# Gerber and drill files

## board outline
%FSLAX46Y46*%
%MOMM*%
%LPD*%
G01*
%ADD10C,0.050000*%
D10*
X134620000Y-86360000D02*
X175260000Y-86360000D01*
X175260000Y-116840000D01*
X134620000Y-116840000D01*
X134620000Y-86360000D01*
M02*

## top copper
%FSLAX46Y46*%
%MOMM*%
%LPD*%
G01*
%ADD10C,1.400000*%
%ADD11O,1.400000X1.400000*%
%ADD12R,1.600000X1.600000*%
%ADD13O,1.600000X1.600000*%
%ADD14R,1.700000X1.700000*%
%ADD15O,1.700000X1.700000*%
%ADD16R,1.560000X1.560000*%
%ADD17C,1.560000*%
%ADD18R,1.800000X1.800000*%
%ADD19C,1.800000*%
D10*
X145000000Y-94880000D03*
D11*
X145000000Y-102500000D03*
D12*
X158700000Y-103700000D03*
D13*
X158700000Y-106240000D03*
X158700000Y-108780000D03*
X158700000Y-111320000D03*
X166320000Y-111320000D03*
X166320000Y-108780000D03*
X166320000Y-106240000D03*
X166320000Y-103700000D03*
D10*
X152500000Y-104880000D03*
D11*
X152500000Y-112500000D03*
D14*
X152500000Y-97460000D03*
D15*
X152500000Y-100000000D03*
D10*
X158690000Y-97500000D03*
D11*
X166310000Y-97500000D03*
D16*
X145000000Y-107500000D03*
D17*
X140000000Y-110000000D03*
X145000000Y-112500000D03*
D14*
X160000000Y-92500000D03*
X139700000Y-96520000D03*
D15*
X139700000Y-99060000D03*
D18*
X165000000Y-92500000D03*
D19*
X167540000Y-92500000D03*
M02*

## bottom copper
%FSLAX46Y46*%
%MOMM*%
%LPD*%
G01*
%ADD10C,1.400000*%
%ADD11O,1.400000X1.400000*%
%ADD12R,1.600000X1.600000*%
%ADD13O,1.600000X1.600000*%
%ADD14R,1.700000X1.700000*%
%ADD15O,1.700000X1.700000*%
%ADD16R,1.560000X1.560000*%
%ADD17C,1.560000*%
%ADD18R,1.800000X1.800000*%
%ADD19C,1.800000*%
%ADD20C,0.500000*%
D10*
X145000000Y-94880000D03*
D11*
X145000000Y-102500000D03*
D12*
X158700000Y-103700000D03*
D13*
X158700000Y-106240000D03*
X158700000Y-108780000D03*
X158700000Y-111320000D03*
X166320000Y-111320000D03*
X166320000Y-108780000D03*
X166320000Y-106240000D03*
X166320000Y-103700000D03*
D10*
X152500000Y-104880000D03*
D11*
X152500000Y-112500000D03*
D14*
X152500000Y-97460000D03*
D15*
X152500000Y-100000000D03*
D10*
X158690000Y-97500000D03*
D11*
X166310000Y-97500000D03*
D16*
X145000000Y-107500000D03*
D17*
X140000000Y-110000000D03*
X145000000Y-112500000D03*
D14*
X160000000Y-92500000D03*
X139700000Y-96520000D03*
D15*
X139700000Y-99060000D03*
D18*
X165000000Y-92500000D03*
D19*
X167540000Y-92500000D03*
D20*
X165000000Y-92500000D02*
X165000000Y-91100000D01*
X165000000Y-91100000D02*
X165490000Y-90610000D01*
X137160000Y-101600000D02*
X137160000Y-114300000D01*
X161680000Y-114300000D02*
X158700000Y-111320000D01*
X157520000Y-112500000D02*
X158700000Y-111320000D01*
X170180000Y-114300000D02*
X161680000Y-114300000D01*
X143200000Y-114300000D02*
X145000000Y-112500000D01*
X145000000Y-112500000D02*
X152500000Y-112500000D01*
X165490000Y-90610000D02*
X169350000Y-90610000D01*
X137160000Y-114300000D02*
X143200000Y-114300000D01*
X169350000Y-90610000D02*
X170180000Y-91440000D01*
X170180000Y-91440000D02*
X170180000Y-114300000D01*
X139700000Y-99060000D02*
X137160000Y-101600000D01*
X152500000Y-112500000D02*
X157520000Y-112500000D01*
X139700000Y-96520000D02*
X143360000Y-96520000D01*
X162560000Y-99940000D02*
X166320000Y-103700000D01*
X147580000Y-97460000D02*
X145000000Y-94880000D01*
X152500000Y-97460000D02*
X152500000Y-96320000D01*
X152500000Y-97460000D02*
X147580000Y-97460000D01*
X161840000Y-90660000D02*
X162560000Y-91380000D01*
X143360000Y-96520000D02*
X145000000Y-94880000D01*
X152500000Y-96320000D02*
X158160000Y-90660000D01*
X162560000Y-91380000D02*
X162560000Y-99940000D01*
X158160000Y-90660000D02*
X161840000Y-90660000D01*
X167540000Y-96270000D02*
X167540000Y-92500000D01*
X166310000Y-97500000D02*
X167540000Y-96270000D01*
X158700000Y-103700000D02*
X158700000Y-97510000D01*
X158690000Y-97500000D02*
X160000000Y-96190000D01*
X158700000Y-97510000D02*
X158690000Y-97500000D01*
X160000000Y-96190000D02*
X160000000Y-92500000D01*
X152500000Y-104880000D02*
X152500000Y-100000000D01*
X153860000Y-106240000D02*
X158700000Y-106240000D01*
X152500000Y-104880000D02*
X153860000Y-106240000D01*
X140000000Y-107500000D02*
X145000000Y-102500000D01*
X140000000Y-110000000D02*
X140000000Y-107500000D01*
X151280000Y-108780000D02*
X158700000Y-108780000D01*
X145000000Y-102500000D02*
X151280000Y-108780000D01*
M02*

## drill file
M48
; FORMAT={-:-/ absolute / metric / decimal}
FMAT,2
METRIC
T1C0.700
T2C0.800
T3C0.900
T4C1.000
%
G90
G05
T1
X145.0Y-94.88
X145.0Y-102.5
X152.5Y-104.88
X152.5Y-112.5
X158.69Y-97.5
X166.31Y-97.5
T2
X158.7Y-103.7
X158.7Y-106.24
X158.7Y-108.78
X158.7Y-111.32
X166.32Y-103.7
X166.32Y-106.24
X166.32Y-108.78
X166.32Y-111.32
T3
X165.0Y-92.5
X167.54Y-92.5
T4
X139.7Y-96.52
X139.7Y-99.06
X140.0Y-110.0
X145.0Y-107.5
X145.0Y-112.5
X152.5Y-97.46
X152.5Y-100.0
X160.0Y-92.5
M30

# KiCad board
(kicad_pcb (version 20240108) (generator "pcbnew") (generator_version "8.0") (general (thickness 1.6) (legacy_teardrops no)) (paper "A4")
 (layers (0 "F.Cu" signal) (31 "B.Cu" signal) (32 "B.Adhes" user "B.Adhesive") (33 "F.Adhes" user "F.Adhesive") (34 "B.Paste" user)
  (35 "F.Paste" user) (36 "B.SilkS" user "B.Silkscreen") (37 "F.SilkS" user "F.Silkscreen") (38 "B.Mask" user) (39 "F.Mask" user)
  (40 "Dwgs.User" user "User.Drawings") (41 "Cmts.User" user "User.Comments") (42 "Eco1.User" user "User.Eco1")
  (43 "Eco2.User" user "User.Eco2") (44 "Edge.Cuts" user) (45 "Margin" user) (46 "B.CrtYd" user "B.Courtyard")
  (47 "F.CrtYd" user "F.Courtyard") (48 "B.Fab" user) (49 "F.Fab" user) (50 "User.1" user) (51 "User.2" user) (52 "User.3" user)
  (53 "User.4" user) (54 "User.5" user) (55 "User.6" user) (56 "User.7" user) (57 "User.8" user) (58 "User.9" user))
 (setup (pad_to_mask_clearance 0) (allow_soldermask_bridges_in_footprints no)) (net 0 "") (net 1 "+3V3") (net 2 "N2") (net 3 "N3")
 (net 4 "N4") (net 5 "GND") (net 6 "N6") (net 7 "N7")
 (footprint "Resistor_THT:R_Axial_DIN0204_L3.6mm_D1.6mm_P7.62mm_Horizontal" (layer "F.Cu") (at 145 94.88 -90)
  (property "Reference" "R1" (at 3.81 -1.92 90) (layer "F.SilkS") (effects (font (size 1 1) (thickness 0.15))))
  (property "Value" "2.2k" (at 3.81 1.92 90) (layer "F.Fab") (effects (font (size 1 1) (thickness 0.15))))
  (pad "1" thru_hole circle (at 0 0 270) (size 1.4 1.4) (drill 0.7) (layers "*.Cu" "*.Mask") (remove_unused_layers no) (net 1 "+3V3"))
  (pad "2" thru_hole oval (at 7.62 0 270) (size 1.4 1.4) (drill 0.7) (layers "*.Cu" "*.Mask") (remove_unused_layers no) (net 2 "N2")))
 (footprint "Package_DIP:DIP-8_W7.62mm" (layer "F.Cu") (at 158.7 103.7)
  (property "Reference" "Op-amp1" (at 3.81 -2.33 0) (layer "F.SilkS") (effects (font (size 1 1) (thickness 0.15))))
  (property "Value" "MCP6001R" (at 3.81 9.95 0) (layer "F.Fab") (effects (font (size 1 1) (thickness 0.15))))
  (pad "1" thru_hole rect (at 0 0) (size 1.6 1.6) (drill 0.8) (layers "*.Cu" "*.Mask") (remove_unused_layers no) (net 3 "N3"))
  (pad "2" thru_hole oval (at 0 2.54) (size 1.6 1.6) (drill 0.8) (layers "*.Cu" "*.Mask") (remove_unused_layers no) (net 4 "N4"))
  (pad "3" thru_hole oval (at 0 5.08) (size 1.6 1.6) (drill 0.8) (layers "*.Cu" "*.Mask") (remove_unused_layers no) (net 2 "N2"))
  (pad "4" thru_hole oval (at 0 7.62) (size 1.6 1.6) (drill 0.8) (layers "*.Cu" "*.Mask") (remove_unused_layers no) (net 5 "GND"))
  (pad "5" thru_hole oval (at 7.62 7.62) (size 1.6 1.6) (drill 0.8) (layers "*.Cu" "*.Mask") (remove_unused_layers no))
  (pad "6" thru_hole oval (at 7.62 5.08) (size 1.6 1.6) (drill 0.8) (layers "*.Cu" "*.Mask") (remove_unused_layers no))
  (pad "7" thru_hole oval (at 7.62 2.54) (size 1.6 1.6) (drill 0.8) (layers "*.Cu" "*.Mask") (remove_unused_layers no))
  (pad "8" thru_hole oval (at 7.62 0) (size 1.6 1.6) (drill 0.8) (layers "*.Cu" "*.Mask") (remove_unused_layers no) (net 1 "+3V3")))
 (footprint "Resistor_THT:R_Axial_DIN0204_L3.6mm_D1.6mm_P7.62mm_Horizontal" (layer "F.Cu") (at 152.5 104.88 -90)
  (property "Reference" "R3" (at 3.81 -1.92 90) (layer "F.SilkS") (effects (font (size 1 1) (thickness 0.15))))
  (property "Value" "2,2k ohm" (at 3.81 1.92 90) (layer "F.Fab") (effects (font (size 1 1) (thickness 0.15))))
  (pad "1" thru_hole circle (at 0 0 270) (size 1.4 1.4) (drill 0.7) (layers "*.Cu" "*.Mask") (remove_unused_layers no) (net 4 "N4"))
  (pad "2" thru_hole oval (at 7.62 0 270) (size 1.4 1.4) (drill 0.7) (layers "*.Cu" "*.Mask") (remove_unused_layers no) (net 5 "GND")))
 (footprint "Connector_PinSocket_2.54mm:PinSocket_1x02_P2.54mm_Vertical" (layer "F.Cu") (at 152.5 97.46)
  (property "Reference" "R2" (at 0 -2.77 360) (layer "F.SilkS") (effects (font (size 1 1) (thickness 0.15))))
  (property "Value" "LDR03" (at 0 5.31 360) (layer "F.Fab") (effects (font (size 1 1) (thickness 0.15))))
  (pad "1" thru_hole rect (at 0 0) (size 1.7 1.7) (drill 1) (layers "*.Cu" "*.Mask") (remove_unused_layers no) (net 1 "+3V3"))
  (pad "2" thru_hole oval (at 0 2.54) (size 1.7 1.7) (drill 1) (layers "*.Cu" "*.Mask") (remove_unused_layers no) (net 4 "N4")))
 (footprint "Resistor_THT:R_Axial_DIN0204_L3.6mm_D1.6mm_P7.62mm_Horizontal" (layer "F.Cu") (at 158.69 97.5)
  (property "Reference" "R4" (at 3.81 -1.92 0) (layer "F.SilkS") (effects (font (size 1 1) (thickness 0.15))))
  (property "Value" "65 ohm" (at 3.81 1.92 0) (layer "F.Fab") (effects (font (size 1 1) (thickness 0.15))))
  (pad "1" thru_hole circle (at 0 0) (size 1.4 1.4) (drill 0.7) (layers "*.Cu" "*.Mask") (remove_unused_layers no) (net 3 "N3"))
  (pad "2" thru_hole oval (at 7.62 0) (size 1.4 1.4) (drill 0.7) (layers "*.Cu" "*.Mask") (remove_unused_layers no) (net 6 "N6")))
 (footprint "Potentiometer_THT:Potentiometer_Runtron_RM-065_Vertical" (layer "F.Cu") (at 145 107.5 -90)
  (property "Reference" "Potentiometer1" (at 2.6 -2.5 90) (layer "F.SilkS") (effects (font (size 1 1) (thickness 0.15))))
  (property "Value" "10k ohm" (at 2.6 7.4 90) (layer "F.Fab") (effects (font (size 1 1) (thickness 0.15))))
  (pad "1" thru_hole rect (at 0 0 270) (size 1.56 1.56) (drill 1) (layers "*.Cu" "*.Mask") (remove_unused_layers no) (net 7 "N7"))
  (pad "2" thru_hole circle (at 2.5 5 270) (size 1.56 1.56) (drill 1) (layers "*.Cu" "*.Mask") (remove_unused_layers no) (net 2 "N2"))
  (pad "3" thru_hole circle (at 5 0 270) (size 1.56 1.56) (drill 1) (layers "*.Cu" "*.Mask") (remove_unused_layers no) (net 5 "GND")))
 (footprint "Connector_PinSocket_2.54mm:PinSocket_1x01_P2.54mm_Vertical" (layer "F.Cu") (at 160 92.5)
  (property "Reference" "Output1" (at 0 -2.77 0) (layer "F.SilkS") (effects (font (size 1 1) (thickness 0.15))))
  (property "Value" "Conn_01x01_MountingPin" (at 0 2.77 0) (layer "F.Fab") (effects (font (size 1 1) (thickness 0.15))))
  (pad "1" thru_hole rect (at 0 0) (size 1.7 1.7) (drill 1) (layers "*.Cu" "*.Mask") (remove_unused_layers no) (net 3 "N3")))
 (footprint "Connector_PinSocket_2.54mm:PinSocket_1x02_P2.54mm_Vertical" (layer "F.Cu") (at 139.7 96.52)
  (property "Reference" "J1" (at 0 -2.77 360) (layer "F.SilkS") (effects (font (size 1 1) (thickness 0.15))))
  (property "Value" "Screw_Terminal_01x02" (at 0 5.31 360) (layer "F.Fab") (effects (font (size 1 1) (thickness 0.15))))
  (pad "1" thru_hole rect (at 0 0) (size 1.7 1.7) (drill 1) (layers "*.Cu" "*.Mask") (remove_unused_layers no) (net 1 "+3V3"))
  (pad "2" thru_hole oval (at 0 2.54) (size 1.7 1.7) (drill 1) (layers "*.Cu" "*.Mask") (remove_unused_layers no) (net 5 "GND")))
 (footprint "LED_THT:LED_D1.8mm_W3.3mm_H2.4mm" (layer "F.Cu") (at 165 92.5)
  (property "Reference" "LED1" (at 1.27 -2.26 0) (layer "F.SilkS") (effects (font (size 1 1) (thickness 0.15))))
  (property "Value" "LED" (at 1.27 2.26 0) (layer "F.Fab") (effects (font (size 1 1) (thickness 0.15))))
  (pad "1" thru_hole rect (at 0 0) (size 1.8 1.8) (drill 0.9) (layers "*.Cu" "*.Mask") (remove_unused_layers no) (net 5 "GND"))
  (pad "2" thru_hole circle (at 2.54 0) (size 1.8 1.8) (drill 0.9) (layers "*.Cu" "*.Mask") (remove_unused_layers no) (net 6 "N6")))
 (gr_rect (start 134.62 86.36) (end 175.26 116.84) (stroke (width 0.05) (type default)) (fill none) (layer "Edge.Cuts"))
 (segment (start 165 92.5) (end 165 91.1) (width 0.5) (layer "B.Cu") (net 5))
 (segment (start 165 91.1) (end 165.49 90.61) (width 0.5) (layer "B.Cu") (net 5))
 (segment (start 137.16 101.6) (end 137.16 114.3) (width 0.5) (layer "B.Cu") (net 5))
 (segment (start 161.68 114.3) (end 158.7 111.32) (width 0.5) (layer "B.Cu") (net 5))
 (segment (start 157.52 112.5) (end 158.7 111.32) (width 0.5) (layer "B.Cu") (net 5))
 (segment (start 170.18 114.3) (end 161.68 114.3) (width 0.5) (layer "B.Cu") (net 5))
 (segment (start 143.2 114.3) (end 145 112.5) (width 0.5) (layer "B.Cu") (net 5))
 (segment (start 145 112.5) (end 152.5 112.5) (width 0.5) (layer "B.Cu") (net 5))
 (segment (start 165.49 90.61) (end 169.35 90.61) (width 0.5) (layer "B.Cu") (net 5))
 (segment (start 137.16 114.3) (end 143.2 114.3) (width 0.5) (layer "B.Cu") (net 5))
 (segment (start 169.35 90.61) (end 170.18 91.44) (width 0.5) (layer "B.Cu") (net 5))
 (segment (start 170.18 91.44) (end 170.18 114.3) (width 0.5) (layer "B.Cu") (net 5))
 (segment (start 139.7 99.06) (end 137.16 101.6) (width 0.5) (layer "B.Cu") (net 5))
 (segment (start 152.5 112.5) (end 157.52 112.5) (width 0.5) (layer "B.Cu") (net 5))
 (segment (start 139.7 96.52) (end 143.36 96.52) (width 0.5) (layer "B.Cu") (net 1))
 (segment (start 162.56 99.94) (end 166.32 103.7) (width 0.5) (layer "B.Cu") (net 1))
 (segment (start 147.58 97.46) (end 145 94.88) (width 0.5) (layer "B.Cu") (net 1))
 (segment (start 152.5 97.46) (end 152.5 96.32) (width 0.5) (layer "B.Cu") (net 1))
 (segment (start 152.5 97.46) (end 147.58 97.46) (width 0.5) (layer "B.Cu") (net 1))
 (segment (start 161.84 90.66) (end 162.56 91.38) (width 0.5) (layer "B.Cu") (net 1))
 (segment (start 143.36 96.52) (end 145 94.88) (width 0.5) (layer "B.Cu") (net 1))
 (segment (start 152.5 96.32) (end 158.16 90.66) (width 0.5) (layer "B.Cu") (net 1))
 (segment (start 162.56 91.38) (end 162.56 99.94) (width 0.5) (layer "B.Cu") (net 1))
 (segment (start 158.16 90.66) (end 161.84 90.66) (width 0.5) (layer "B.Cu") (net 1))
 (segment (start 167.54 96.27) (end 167.54 92.5) (width 0.5) (layer "B.Cu") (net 6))
 (segment (start 166.31 97.5) (end 167.54 96.27) (width 0.5) (layer "B.Cu") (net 6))
 (segment (start 158.7 103.7) (end 158.7 97.51) (width 0.5) (layer "B.Cu") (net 3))
 (segment (start 158.69 97.5) (end 160 96.19) (width 0.5) (layer "B.Cu") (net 3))
 (segment (start 158.7 97.51) (end 158.69 97.5) (width 0.5) (layer "B.Cu") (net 3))
 (segment (start 160 96.19) (end 160 92.5) (width 0.5) (layer "B.Cu") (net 3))
 (segment (start 152.5 104.88) (end 152.5 100) (width 0.5) (layer "B.Cu") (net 4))
 (segment (start 153.86 106.24) (end 158.7 106.24) (width 0.5) (layer "B.Cu") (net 4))
 (segment (start 152.5 104.88) (end 153.86 106.24) (width 0.5) (layer "B.Cu") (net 4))
 (segment (start 140 107.5) (end 145 102.5) (width 0.5) (layer "B.Cu") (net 2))
 (segment (start 140 110) (end 140 107.5) (width 0.5) (layer "B.Cu") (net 2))
 (segment (start 151.28 108.78) (end 158.7 108.78) (width 0.5) (layer "B.Cu") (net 2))
 (segment (start 145 102.5) (end 151.28 108.78) (width 0.5) (layer "B.Cu") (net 2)))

